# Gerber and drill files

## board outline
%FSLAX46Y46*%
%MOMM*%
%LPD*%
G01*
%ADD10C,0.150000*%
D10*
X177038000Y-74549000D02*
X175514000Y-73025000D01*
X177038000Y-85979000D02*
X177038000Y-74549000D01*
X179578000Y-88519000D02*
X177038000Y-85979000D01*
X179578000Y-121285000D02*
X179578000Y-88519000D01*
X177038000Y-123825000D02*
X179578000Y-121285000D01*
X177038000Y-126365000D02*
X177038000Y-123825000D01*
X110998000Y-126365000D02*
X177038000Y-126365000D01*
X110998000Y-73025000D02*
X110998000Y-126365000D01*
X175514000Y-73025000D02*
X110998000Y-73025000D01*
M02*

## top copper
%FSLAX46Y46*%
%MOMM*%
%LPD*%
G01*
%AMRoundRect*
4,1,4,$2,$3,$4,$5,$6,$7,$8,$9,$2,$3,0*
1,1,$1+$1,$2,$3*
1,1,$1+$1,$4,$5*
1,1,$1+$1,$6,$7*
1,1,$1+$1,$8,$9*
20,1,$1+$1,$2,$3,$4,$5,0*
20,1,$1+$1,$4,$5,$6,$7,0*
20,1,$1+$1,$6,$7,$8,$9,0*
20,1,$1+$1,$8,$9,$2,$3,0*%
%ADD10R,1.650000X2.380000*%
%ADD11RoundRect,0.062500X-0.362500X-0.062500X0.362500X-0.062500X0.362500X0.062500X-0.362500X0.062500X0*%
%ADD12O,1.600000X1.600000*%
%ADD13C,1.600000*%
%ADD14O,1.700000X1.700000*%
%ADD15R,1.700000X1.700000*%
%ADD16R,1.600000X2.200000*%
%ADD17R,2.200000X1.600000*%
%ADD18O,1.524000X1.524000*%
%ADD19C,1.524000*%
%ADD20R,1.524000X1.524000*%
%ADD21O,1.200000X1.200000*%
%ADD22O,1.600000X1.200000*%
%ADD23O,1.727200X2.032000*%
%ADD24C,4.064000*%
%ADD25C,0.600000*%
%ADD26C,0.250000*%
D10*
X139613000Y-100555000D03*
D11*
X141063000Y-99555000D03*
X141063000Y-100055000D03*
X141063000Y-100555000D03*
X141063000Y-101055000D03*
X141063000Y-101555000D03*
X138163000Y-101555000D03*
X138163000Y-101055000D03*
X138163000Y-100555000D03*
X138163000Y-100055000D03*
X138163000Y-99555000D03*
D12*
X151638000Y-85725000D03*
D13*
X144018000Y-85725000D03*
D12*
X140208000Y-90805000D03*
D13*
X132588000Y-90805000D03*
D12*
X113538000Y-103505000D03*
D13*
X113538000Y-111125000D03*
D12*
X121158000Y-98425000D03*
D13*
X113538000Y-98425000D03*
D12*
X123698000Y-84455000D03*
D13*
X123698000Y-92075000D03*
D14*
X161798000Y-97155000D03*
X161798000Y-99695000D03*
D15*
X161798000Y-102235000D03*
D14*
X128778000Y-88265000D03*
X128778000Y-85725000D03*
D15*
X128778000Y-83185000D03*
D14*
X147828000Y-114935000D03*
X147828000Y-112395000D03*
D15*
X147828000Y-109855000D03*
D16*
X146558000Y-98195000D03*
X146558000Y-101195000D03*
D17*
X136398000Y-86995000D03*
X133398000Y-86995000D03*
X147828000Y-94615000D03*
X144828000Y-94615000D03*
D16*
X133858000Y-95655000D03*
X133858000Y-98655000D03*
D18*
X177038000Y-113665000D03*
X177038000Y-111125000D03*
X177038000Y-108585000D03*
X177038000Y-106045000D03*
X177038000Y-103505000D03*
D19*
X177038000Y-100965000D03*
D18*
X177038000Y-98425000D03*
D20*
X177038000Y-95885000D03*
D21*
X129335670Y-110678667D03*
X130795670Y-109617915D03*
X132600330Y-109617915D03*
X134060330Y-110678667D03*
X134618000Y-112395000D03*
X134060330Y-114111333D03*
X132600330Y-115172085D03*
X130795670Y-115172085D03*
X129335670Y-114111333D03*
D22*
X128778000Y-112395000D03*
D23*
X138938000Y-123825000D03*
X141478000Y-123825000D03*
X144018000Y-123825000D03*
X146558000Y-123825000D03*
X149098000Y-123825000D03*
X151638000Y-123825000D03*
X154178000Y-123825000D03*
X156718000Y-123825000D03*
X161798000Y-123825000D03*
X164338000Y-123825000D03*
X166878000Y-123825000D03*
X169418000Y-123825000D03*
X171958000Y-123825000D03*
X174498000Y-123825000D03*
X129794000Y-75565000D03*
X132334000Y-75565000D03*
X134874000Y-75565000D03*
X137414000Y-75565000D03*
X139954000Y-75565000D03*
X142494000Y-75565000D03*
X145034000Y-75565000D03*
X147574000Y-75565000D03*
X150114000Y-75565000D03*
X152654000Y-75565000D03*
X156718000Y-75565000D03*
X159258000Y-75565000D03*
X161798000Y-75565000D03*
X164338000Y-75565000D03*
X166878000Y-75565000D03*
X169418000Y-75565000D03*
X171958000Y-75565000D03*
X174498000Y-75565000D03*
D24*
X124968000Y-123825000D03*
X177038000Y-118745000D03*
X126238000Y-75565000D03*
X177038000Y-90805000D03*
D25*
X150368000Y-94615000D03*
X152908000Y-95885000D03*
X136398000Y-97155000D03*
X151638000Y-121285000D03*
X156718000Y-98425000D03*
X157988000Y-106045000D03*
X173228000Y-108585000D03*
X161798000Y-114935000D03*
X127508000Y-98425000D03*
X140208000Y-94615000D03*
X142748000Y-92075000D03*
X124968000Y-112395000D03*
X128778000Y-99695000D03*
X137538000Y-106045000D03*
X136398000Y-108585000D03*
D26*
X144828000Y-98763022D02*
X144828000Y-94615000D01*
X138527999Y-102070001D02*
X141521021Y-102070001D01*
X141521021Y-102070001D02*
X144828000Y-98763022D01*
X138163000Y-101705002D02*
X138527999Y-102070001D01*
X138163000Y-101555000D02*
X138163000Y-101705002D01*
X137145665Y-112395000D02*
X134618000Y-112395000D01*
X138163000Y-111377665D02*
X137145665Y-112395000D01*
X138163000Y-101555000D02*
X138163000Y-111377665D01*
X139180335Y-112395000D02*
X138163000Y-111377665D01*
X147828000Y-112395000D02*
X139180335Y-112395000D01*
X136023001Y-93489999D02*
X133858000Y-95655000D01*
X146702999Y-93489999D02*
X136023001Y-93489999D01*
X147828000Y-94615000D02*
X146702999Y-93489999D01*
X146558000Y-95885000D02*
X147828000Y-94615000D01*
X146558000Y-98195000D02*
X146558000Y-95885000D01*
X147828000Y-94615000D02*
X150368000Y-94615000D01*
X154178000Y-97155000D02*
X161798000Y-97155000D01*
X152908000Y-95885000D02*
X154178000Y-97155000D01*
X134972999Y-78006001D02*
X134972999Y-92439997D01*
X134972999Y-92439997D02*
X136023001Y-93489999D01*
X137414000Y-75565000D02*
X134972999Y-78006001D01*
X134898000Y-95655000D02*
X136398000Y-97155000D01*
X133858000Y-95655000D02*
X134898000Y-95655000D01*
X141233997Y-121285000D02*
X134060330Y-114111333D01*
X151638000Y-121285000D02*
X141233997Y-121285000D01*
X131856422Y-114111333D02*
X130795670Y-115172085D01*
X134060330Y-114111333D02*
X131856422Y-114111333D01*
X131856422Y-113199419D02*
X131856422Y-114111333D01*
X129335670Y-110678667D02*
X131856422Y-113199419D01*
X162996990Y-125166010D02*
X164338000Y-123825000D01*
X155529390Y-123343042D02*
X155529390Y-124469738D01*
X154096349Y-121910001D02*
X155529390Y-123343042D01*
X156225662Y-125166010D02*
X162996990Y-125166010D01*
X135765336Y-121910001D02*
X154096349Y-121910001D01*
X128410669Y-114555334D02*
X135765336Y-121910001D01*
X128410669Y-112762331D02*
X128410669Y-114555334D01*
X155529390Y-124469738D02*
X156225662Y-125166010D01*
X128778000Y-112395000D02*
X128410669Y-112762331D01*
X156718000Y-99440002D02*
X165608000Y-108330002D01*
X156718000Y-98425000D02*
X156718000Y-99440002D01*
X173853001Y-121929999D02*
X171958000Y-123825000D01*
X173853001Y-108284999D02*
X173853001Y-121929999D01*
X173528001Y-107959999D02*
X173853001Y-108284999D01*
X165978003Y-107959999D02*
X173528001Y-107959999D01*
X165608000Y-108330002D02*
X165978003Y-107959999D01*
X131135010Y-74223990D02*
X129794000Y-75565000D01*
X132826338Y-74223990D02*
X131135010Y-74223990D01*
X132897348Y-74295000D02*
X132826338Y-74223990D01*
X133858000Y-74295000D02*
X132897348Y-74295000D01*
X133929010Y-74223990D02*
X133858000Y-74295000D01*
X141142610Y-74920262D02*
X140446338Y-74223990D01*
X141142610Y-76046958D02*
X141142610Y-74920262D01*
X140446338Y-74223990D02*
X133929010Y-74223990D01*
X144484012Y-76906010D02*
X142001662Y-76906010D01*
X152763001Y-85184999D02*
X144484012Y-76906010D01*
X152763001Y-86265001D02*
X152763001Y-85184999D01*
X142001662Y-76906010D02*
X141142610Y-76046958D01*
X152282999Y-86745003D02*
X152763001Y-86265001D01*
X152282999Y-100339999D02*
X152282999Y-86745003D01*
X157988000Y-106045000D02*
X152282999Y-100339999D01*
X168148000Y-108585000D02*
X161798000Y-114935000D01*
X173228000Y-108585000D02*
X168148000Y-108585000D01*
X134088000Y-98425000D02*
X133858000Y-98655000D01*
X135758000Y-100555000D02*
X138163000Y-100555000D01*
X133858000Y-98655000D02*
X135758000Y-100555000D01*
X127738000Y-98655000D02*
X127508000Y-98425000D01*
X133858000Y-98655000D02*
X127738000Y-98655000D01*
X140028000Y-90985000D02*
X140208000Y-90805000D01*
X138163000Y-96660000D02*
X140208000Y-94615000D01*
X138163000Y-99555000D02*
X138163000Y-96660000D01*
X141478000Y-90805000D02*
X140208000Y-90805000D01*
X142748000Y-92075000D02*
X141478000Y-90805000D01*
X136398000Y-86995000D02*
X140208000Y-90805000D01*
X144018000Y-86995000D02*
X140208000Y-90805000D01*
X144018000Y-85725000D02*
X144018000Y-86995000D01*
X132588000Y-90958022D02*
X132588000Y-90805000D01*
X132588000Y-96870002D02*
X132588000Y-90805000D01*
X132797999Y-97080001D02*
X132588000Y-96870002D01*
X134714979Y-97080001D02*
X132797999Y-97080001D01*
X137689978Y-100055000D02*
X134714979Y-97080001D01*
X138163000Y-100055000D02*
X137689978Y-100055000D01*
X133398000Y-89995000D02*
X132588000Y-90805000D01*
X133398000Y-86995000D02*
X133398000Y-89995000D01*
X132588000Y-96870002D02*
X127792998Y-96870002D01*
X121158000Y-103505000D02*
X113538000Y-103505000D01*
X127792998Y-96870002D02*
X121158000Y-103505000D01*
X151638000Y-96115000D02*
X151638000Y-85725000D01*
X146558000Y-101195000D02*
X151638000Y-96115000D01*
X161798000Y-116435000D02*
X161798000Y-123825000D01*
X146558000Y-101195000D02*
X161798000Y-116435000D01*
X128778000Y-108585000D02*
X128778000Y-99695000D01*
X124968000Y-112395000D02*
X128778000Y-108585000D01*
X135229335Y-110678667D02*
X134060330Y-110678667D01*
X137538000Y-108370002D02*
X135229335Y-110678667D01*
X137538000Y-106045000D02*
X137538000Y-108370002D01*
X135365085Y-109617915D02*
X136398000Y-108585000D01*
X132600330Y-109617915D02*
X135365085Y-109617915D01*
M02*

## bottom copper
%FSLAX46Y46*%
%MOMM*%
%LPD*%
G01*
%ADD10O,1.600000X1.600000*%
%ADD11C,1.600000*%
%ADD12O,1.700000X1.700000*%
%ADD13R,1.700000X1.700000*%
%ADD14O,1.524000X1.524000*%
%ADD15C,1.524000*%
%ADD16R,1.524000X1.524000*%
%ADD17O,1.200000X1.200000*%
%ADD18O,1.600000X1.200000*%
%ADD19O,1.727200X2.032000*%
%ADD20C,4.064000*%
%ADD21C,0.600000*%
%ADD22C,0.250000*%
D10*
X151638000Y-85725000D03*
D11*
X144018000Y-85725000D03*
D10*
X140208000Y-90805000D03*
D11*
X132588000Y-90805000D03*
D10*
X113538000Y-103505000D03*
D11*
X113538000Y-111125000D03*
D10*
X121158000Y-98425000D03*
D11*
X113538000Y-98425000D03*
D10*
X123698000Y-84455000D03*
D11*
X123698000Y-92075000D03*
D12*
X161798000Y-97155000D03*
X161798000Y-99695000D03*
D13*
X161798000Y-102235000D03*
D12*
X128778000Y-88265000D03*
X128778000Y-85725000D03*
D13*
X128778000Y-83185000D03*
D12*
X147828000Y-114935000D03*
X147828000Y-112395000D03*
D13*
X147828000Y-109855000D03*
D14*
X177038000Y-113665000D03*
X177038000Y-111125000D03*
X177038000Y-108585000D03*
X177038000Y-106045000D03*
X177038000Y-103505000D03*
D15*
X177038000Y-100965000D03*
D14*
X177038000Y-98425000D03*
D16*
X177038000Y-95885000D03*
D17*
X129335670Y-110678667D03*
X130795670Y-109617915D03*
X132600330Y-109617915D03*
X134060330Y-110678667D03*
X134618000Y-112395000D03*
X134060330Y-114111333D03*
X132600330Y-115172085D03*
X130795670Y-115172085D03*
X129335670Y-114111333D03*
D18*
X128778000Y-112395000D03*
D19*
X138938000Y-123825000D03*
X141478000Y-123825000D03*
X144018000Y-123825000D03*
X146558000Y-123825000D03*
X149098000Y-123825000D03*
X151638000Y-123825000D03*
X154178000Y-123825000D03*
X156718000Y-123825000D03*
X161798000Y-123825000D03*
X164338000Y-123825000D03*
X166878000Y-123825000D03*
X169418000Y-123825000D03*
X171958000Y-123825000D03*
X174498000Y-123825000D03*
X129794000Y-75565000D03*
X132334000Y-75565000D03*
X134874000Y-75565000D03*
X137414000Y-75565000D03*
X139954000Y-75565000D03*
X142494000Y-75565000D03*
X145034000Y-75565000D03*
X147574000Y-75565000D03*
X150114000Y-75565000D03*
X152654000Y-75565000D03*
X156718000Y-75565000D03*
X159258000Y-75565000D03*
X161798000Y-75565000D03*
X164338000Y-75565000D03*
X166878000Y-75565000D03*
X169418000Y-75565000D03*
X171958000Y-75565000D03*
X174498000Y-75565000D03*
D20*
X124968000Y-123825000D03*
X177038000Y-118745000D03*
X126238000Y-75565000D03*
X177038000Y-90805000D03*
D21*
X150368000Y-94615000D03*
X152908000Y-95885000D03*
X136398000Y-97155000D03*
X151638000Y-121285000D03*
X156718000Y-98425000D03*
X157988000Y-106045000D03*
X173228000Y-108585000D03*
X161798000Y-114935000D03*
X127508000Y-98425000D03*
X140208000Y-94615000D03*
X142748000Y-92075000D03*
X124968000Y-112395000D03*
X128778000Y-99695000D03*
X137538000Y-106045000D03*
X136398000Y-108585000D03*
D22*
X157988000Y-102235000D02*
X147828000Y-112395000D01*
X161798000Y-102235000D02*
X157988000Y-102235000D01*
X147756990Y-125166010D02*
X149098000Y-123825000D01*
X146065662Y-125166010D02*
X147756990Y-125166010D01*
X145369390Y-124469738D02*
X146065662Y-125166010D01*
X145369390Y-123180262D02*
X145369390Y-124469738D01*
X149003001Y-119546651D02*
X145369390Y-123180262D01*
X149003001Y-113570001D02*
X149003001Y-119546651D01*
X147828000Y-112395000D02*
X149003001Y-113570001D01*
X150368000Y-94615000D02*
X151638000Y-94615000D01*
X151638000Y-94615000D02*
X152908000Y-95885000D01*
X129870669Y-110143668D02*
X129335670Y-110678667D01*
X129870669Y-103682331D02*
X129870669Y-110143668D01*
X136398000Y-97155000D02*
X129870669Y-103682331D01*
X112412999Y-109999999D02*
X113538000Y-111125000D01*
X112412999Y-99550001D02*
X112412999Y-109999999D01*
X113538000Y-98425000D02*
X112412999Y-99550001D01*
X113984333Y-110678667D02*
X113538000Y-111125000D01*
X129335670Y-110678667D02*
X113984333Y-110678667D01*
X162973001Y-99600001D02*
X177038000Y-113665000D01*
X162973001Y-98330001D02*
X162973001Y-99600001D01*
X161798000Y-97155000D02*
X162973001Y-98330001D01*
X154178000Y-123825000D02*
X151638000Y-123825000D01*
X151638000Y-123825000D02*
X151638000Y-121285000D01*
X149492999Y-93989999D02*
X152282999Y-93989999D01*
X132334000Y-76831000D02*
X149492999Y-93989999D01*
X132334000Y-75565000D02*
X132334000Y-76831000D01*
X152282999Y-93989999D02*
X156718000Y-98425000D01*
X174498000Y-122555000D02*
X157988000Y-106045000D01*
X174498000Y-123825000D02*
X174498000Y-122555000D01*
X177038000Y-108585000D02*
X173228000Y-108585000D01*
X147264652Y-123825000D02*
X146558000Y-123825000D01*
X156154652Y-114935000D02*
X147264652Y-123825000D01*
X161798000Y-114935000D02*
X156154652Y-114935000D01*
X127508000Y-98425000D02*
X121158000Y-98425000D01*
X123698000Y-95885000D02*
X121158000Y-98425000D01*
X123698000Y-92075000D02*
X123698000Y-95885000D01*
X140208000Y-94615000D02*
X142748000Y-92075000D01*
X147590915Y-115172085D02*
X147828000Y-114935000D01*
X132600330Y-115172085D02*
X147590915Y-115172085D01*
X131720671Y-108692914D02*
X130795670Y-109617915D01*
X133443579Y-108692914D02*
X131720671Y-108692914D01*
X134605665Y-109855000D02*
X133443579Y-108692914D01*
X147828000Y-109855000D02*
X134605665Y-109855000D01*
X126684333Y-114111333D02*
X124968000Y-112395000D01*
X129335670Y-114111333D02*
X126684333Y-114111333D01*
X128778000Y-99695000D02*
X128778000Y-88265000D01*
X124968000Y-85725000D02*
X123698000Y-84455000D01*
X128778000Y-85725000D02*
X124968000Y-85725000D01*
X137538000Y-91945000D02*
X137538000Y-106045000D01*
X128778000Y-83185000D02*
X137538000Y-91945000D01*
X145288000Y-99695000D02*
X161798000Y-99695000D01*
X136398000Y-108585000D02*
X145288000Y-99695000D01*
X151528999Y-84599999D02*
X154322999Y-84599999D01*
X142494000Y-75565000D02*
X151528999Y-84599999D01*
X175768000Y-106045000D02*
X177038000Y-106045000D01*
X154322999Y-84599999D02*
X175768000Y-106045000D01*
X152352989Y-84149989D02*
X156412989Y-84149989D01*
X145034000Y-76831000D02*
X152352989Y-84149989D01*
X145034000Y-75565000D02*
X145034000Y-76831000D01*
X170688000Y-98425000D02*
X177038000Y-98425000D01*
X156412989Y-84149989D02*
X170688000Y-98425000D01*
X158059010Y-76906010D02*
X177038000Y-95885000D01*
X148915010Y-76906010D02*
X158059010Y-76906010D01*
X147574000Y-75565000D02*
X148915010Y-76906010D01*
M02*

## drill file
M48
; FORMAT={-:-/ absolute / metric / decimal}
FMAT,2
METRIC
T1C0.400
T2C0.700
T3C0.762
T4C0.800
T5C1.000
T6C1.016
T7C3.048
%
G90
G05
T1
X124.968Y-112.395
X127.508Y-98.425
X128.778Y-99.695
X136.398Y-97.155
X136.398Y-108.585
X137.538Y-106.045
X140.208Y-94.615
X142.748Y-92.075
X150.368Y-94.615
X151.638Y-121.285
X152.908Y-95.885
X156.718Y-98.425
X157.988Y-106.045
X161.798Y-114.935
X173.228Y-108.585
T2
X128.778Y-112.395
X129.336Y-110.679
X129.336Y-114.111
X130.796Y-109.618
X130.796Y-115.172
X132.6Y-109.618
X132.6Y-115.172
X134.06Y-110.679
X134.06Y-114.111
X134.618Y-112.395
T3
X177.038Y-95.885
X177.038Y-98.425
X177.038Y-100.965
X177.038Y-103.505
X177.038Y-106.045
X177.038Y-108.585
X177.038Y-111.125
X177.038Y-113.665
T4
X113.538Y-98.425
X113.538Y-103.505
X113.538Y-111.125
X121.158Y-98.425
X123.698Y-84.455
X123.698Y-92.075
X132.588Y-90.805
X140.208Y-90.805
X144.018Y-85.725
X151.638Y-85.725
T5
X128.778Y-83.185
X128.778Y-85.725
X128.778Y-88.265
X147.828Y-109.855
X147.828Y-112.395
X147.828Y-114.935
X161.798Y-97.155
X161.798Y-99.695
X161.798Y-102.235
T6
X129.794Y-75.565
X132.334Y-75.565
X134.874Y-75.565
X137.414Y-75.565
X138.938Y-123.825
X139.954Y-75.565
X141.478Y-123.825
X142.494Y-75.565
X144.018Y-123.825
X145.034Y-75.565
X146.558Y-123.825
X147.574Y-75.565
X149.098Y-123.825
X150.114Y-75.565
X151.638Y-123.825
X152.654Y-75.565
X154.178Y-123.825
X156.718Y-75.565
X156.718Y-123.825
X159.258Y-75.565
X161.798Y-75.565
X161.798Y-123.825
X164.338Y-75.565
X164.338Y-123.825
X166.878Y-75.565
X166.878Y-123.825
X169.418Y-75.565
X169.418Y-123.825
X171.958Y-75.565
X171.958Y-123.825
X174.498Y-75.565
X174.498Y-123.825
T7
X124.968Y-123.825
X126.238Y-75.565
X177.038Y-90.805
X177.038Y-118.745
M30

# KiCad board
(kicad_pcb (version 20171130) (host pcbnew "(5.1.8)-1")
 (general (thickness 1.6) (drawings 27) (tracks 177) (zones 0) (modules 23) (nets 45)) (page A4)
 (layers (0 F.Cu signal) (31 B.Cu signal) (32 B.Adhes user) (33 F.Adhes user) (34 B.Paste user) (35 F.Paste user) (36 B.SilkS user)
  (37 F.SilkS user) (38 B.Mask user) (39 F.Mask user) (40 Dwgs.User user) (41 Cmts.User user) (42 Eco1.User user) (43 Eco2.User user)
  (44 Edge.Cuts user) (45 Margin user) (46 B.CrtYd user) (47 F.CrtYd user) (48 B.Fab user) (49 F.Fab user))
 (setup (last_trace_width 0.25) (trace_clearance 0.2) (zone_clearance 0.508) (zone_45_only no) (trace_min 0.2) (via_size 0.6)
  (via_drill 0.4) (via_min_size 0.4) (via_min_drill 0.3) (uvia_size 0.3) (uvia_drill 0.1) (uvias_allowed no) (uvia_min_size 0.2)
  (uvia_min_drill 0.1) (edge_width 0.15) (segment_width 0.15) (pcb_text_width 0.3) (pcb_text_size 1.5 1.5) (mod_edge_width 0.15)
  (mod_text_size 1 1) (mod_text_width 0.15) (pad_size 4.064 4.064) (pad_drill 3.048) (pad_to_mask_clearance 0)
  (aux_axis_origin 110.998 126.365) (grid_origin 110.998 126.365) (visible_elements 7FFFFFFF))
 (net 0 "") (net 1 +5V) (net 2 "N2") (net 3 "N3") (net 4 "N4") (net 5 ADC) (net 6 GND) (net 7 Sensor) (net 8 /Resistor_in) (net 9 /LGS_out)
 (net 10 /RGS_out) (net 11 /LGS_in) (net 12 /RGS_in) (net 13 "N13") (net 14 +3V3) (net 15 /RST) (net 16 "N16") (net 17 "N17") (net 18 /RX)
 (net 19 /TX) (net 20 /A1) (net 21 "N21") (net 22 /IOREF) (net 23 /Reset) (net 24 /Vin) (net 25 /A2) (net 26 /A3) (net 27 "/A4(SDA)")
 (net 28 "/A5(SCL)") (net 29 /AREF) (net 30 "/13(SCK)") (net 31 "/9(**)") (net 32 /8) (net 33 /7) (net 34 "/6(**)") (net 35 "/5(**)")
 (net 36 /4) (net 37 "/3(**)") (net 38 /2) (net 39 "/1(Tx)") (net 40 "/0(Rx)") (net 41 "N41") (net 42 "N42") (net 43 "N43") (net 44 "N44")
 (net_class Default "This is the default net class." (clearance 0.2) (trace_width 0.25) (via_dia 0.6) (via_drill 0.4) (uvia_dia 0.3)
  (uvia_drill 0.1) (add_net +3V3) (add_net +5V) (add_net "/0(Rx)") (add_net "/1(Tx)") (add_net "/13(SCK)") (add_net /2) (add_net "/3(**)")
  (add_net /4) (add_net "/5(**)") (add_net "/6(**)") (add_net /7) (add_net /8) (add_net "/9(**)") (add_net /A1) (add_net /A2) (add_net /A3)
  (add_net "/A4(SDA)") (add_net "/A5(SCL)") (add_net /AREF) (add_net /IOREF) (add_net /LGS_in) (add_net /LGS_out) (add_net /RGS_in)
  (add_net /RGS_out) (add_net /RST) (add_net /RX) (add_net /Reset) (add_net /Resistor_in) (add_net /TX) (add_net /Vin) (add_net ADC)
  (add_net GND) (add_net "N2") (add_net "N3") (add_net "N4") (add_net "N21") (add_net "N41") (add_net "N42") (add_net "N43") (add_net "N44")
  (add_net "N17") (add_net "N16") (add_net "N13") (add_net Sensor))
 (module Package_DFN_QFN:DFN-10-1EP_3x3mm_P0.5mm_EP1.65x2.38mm (layer F.Cu) (at 139.613 100.555)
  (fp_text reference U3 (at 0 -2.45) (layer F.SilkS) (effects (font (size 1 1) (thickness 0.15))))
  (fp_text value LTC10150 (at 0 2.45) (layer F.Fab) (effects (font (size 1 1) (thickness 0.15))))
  (pad "" smd roundrect (at 0.41 0.595) (size 0.67 0.96) (layers F.Paste) (roundrect_rratio 0.25))
  (pad "" smd roundrect (at 0.41 -0.595) (size 0.67 0.96) (layers F.Paste) (roundrect_rratio 0.25))
  (pad "" smd roundrect (at -0.41 0.595) (size 0.67 0.96) (layers F.Paste) (roundrect_rratio 0.25))
  (pad "" smd roundrect (at -0.41 -0.595) (size 0.67 0.96) (layers F.Paste) (roundrect_rratio 0.25))
  (pad 11 smd rect (at 0 0) (size 1.65 2.38) (layers F.Cu F.Mask))
  (pad 10 smd roundrect (at 1.45 -1) (size 0.85 0.25) (layers F.Cu F.Paste F.Mask) (roundrect_rratio 0.25))
  (pad 9 smd roundrect (at 1.45 -0.5) (size 0.85 0.25) (layers F.Cu F.Paste F.Mask) (roundrect_rratio 0.25))
  (pad 8 smd roundrect (at 1.45 0) (size 0.85 0.25) (layers F.Cu F.Paste F.Mask) (roundrect_rratio 0.25))
  (pad 7 smd roundrect (at 1.45 0.5) (size 0.85 0.25) (layers F.Cu F.Paste F.Mask) (roundrect_rratio 0.25))
  (pad 6 smd roundrect (at 1.45 1) (size 0.85 0.25) (layers F.Cu F.Paste F.Mask) (roundrect_rratio 0.25))
  (pad 5 smd roundrect (at -1.45 1) (size 0.85 0.25) (layers F.Cu F.Paste F.Mask) (roundrect_rratio 0.25) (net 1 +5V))
  (pad 4 smd roundrect (at -1.45 0.5) (size 0.85 0.25) (layers F.Cu F.Paste F.Mask) (roundrect_rratio 0.25))
  (pad 3 smd roundrect (at -1.45 0) (size 0.85 0.25) (layers F.Cu F.Paste F.Mask) (roundrect_rratio 0.25) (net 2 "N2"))
  (pad 2 smd roundrect (at -1.45 -0.5) (size 0.85 0.25) (layers F.Cu F.Paste F.Mask) (roundrect_rratio 0.25) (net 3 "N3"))
  (pad 1 smd roundrect (at -1.45 -1) (size 0.85 0.25) (layers F.Cu F.Paste F.Mask) (roundrect_rratio 0.25) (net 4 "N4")))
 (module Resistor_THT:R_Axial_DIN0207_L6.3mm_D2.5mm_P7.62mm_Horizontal (layer F.Cu) (at 144.018 85.725)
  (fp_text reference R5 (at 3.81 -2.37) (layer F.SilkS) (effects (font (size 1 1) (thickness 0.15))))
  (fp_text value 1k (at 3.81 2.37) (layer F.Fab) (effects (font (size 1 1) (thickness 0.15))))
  (pad 2 thru_hole oval (at 7.62 0) (size 1.6 1.6) (drill 0.8) (layers *.Cu *.Mask) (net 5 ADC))
  (pad 1 thru_hole circle (at 0 0) (size 1.6 1.6) (drill 0.8) (layers *.Cu *.Mask) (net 4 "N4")))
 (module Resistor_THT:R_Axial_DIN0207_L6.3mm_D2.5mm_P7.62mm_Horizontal (layer F.Cu) (at 132.588 90.805)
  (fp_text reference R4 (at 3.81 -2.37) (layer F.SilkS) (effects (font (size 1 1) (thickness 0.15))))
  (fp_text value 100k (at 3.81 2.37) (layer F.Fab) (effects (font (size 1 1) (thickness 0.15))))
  (pad 2 thru_hole oval (at 7.62 0) (size 1.6 1.6) (drill 0.8) (layers *.Cu *.Mask) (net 4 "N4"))
  (pad 1 thru_hole circle (at 0 0) (size 1.6 1.6) (drill 0.8) (layers *.Cu *.Mask) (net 3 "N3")))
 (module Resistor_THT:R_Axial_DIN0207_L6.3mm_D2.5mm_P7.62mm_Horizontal (layer F.Cu) (at 113.538 111.125 90)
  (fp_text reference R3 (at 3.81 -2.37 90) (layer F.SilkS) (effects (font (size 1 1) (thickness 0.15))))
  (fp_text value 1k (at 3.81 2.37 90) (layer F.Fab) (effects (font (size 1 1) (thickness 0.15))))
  (pad 2 thru_hole oval (at 7.62 0 90) (size 1.6 1.6) (drill 0.8) (layers *.Cu *.Mask) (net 3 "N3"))
  (pad 1 thru_hole circle (at 0 0 90) (size 1.6 1.6) (drill 0.8) (layers *.Cu *.Mask) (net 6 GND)))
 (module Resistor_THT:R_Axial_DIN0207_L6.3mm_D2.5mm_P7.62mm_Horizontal (layer F.Cu) (at 113.538 98.425)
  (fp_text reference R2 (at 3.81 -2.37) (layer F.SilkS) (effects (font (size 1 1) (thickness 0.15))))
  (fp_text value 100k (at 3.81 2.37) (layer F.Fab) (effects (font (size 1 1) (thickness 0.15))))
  (pad 2 thru_hole oval (at 7.62 0) (size 1.6 1.6) (drill 0.8) (layers *.Cu *.Mask) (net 2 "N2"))
  (pad 1 thru_hole circle (at 0 0) (size 1.6 1.6) (drill 0.8) (layers *.Cu *.Mask) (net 6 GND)))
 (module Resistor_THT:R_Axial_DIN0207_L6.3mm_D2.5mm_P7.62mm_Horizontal (layer F.Cu) (at 123.698 92.075 90)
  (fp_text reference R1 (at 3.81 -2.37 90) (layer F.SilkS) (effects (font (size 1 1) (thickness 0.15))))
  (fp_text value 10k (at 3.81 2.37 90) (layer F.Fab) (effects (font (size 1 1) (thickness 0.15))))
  (pad 2 thru_hole oval (at 7.62 0 90) (size 1.6 1.6) (drill 0.8) (layers *.Cu *.Mask) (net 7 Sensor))
  (pad 1 thru_hole circle (at 0 0 90) (size 1.6 1.6) (drill 0.8) (layers *.Cu *.Mask) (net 2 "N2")))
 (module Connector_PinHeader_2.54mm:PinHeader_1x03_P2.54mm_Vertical (layer F.Cu) (at 161.798 102.235 180)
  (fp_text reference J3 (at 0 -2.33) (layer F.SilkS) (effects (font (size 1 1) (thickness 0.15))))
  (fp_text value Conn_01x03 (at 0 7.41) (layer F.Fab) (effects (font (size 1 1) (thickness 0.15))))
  (pad 3 thru_hole oval (at 0 5.08 180) (size 1.7 1.7) (drill 1) (layers *.Cu *.Mask) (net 6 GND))
  (pad 2 thru_hole oval (at 0 2.54 180) (size 1.7 1.7) (drill 1) (layers *.Cu *.Mask) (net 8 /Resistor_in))
  (pad 1 thru_hole rect (at 0 0 180) (size 1.7 1.7) (drill 1) (layers *.Cu *.Mask) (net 1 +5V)))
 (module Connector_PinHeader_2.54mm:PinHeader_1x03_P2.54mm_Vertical (layer F.Cu) (at 128.778 83.185)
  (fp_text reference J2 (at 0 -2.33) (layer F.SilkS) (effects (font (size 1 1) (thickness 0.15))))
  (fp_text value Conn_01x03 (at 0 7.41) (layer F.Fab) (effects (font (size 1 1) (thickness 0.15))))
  (pad 3 thru_hole oval (at 0 5.08) (size 1.7 1.7) (drill 1) (layers *.Cu *.Mask) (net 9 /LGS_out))
  (pad 2 thru_hole oval (at 0 2.54) (size 1.7 1.7) (drill 1) (layers *.Cu *.Mask) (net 7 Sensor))
  (pad 1 thru_hole rect (at 0 0) (size 1.7 1.7) (drill 1) (layers *.Cu *.Mask) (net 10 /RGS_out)))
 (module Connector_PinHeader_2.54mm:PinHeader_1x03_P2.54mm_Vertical (layer F.Cu) (at 147.828 109.855)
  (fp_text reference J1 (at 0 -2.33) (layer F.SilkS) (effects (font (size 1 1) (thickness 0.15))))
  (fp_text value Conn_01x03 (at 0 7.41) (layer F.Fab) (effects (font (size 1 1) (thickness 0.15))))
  (pad 3 thru_hole oval (at 0 5.08) (size 1.7 1.7) (drill 1) (layers *.Cu *.Mask) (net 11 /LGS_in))
  (pad 2 thru_hole oval (at 0 2.54) (size 1.7 1.7) (drill 1) (layers *.Cu *.Mask) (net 1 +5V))
  (pad 1 thru_hole rect (at 0 0) (size 1.7 1.7) (drill 1) (layers *.Cu *.Mask) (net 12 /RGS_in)))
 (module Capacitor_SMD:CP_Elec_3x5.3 (layer F.Cu) (at 146.558 99.695 90)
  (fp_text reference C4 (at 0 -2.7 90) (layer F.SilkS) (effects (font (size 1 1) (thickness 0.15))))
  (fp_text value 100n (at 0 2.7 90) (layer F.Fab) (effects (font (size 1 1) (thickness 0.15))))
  (pad 2 smd rect (at 1.5 0 90) (size 2.2 1.6) (layers F.Cu F.Paste F.Mask) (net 6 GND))
  (pad 1 smd rect (at -1.5 0 90) (size 2.2 1.6) (layers F.Cu F.Paste F.Mask) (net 5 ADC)))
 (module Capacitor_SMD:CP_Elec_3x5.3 (layer F.Cu) (at 134.898 86.995)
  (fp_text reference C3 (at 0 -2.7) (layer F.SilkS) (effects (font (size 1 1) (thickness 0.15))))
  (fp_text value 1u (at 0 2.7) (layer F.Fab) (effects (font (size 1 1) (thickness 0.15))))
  (pad 2 smd rect (at 1.5 0) (size 2.2 1.6) (layers F.Cu F.Paste F.Mask) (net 4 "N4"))
  (pad 1 smd rect (at -1.5 0) (size 2.2 1.6) (layers F.Cu F.Paste F.Mask) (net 3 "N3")))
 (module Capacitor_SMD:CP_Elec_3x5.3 (layer F.Cu) (at 146.328 94.615)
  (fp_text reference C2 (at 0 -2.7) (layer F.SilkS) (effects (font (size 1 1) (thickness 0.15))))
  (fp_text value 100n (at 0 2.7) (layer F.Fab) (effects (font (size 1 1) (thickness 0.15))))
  (pad 2 smd rect (at 1.5 0) (size 2.2 1.6) (layers F.Cu F.Paste F.Mask) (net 6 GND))
  (pad 1 smd rect (at -1.5 0) (size 2.2 1.6) (layers F.Cu F.Paste F.Mask) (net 1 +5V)))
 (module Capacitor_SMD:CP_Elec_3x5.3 (layer F.Cu) (at 133.858 97.155 90)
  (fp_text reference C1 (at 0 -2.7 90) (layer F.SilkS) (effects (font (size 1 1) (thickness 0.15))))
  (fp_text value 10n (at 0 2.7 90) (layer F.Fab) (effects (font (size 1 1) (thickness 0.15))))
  (pad 2 smd rect (at 1.5 0 90) (size 2.2 1.6) (layers F.Cu F.Paste F.Mask) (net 6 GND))
  (pad 1 smd rect (at -1.5 0 90) (size 2.2 1.6) (layers F.Cu F.Paste F.Mask) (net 2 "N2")))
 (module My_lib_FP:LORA (layer F.Cu) (at 197.358 106.045 270)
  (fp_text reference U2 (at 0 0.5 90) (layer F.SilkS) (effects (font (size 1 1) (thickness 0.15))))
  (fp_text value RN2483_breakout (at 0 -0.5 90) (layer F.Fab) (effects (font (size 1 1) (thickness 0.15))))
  (pad 8 thru_hole oval (at 7.62 20.32 270) (size 1.524 1.524) (drill 0.762) (layers *.Cu *.Mask) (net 6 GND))
  (pad 7 thru_hole oval (at 5.08 20.32 270) (size 1.524 1.524) (drill 0.762) (layers *.Cu *.Mask) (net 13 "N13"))
  (pad 6 thru_hole oval (at 2.54 20.32 270) (size 1.524 1.524) (drill 0.762) (layers *.Cu *.Mask) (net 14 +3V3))
  (pad 5 thru_hole oval (at 0 20.32 270) (size 1.524 1.524) (drill 0.762) (layers *.Cu *.Mask) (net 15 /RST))
  (pad 4 thru_hole oval (at -2.54 20.32 270) (size 1.524 1.524) (drill 0.762) (layers *.Cu *.Mask) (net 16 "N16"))
  (pad 3 thru_hole circle (at -5.08 20.32 270) (size 1.524 1.524) (drill 0.762) (layers *.Cu *.Mask) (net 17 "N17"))
  (pad 2 thru_hole oval (at -7.62 20.32 270) (size 1.524 1.524) (drill 0.762) (layers *.Cu *.Mask B.Adhes) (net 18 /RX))
  (pad 1 thru_hole rect (at -10.16 20.32 270) (size 1.524 1.524) (drill 0.762) (layers *.Cu *.Mask) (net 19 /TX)))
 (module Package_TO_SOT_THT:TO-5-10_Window (layer F.Cu) (at 128.778 112.395)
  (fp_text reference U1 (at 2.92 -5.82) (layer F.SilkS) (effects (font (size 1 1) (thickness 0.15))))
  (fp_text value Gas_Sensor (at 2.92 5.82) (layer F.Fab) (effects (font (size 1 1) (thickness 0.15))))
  (pad 10 thru_hole oval (at 0.55767 -1.716333) (size 1.2 1.2) (drill 0.7) (layers *.Cu *.Mask) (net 6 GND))
  (pad 9 thru_hole oval (at 2.01767 -2.777085) (size 1.2 1.2) (drill 0.7) (layers *.Cu *.Mask) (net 12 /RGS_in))
  (pad 8 thru_hole oval (at 3.82233 -2.777085) (size 1.2 1.2) (drill 0.7) (layers *.Cu *.Mask) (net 8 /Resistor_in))
  (pad 7 thru_hole oval (at 5.28233 -1.716333) (size 1.2 1.2) (drill 0.7) (layers *.Cu *.Mask) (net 10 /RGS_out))
  (pad 6 thru_hole oval (at 5.84 0) (size 1.2 1.2) (drill 0.7) (layers *.Cu *.Mask) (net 1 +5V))
  (pad 5 thru_hole oval (at 5.28233 1.716333) (size 1.2 1.2) (drill 0.7) (layers *.Cu *.Mask) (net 6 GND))
  (pad 4 thru_hole oval (at 3.82233 2.777085) (size 1.2 1.2) (drill 0.7) (layers *.Cu *.Mask) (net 11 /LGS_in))
  (pad 3 thru_hole oval (at 2.01767 2.777085) (size 1.2 1.2) (drill 0.7) (layers *.Cu *.Mask) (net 6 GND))
  (pad 2 thru_hole oval (at 0.55767 1.716333) (size 1.2 1.2) (drill 0.7) (layers *.Cu *.Mask) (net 9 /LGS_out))
  (pad 1 thru_hole oval (at 0 0) (size 1.6 1.2) (drill 0.7) (layers *.Cu *.Mask) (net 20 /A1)))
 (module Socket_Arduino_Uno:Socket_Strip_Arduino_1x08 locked (layer F.Cu) (at 138.938 123.825)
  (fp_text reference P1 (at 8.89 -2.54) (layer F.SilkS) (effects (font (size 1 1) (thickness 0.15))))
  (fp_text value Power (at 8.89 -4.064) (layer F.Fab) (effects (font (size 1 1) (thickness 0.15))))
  (pad 1 thru_hole oval (at 0 0) (size 1.7272 2.032) (drill 1.016) (layers *.Cu *.Mask F.SilkS) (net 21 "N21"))
  (pad 2 thru_hole oval (at 2.54 0) (size 1.7272 2.032) (drill 1.016) (layers *.Cu *.Mask F.SilkS) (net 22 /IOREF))
  (pad 3 thru_hole oval (at 5.08 0) (size 1.7272 2.032) (drill 1.016) (layers *.Cu *.Mask F.SilkS) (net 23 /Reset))
  (pad 4 thru_hole oval (at 7.62 0) (size 1.7272 2.032) (drill 1.016) (layers *.Cu *.Mask F.SilkS) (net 14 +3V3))
  (pad 5 thru_hole oval (at 10.16 0) (size 1.7272 2.032) (drill 1.016) (layers *.Cu *.Mask F.SilkS) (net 1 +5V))
  (pad 6 thru_hole oval (at 12.7 0) (size 1.7272 2.032) (drill 1.016) (layers *.Cu *.Mask F.SilkS) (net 6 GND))
  (pad 7 thru_hole oval (at 15.24 0) (size 1.7272 2.032) (drill 1.016) (layers *.Cu *.Mask F.SilkS) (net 6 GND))
  (pad 8 thru_hole oval (at 17.78 0) (size 1.7272 2.032) (drill 1.016) (layers *.Cu *.Mask F.SilkS) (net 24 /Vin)))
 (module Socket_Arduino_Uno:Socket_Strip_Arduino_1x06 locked (layer F.Cu) (at 161.798 123.825)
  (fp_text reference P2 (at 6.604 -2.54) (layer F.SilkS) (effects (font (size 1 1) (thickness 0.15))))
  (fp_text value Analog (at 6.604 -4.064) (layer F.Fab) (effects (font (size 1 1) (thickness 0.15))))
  (pad 1 thru_hole oval (at 0 0) (size 1.7272 2.032) (drill 1.016) (layers *.Cu *.Mask F.SilkS) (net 5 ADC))
  (pad 2 thru_hole oval (at 2.54 0) (size 1.7272 2.032) (drill 1.016) (layers *.Cu *.Mask F.SilkS) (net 20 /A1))
  (pad 3 thru_hole oval (at 5.08 0) (size 1.7272 2.032) (drill 1.016) (layers *.Cu *.Mask F.SilkS) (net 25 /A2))
  (pad 4 thru_hole oval (at 7.62 0) (size 1.7272 2.032) (drill 1.016) (layers *.Cu *.Mask F.SilkS) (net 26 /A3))
  (pad 5 thru_hole oval (at 10.16 0) (size 1.7272 2.032) (drill 1.016) (layers *.Cu *.Mask F.SilkS) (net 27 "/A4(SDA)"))
  (pad 6 thru_hole oval (at 12.7 0) (size 1.7272 2.032) (drill 1.016) (layers *.Cu *.Mask F.SilkS) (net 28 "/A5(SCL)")))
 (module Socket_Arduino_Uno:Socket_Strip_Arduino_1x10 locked (layer F.Cu) (at 129.794 75.565)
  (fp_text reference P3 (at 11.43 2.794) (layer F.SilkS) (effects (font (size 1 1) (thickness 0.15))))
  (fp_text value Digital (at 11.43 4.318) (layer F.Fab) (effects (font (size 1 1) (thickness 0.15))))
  (pad 1 thru_hole oval (at 0 0) (size 1.7272 2.032) (drill 1.016) (layers *.Cu *.Mask F.SilkS) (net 28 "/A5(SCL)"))
  (pad 2 thru_hole oval (at 2.54 0) (size 1.7272 2.032) (drill 1.016) (layers *.Cu *.Mask F.SilkS) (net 27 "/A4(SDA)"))
  (pad 3 thru_hole oval (at 5.08 0) (size 1.7272 2.032) (drill 1.016) (layers *.Cu *.Mask F.SilkS) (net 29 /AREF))
  (pad 4 thru_hole oval (at 7.62 0) (size 1.7272 2.032) (drill 1.016) (layers *.Cu *.Mask F.SilkS) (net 6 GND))
  (pad 5 thru_hole oval (at 10.16 0) (size 1.7272 2.032) (drill 1.016) (layers *.Cu *.Mask F.SilkS) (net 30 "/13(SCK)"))
  (pad 6 thru_hole oval (at 12.7 0) (size 1.7272 2.032) (drill 1.016) (layers *.Cu *.Mask F.SilkS) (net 15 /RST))
  (pad 7 thru_hole oval (at 15.24 0) (size 1.7272 2.032) (drill 1.016) (layers *.Cu *.Mask F.SilkS) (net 18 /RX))
  (pad 8 thru_hole oval (at 17.78 0) (size 1.7272 2.032) (drill 1.016) (layers *.Cu *.Mask F.SilkS) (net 19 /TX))
  (pad 9 thru_hole oval (at 20.32 0) (size 1.7272 2.032) (drill 1.016) (layers *.Cu *.Mask F.SilkS) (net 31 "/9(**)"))
  (pad 10 thru_hole oval (at 22.86 0) (size 1.7272 2.032) (drill 1.016) (layers *.Cu *.Mask F.SilkS) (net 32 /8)))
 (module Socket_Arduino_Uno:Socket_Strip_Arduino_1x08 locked (layer F.Cu) (at 156.718 75.565)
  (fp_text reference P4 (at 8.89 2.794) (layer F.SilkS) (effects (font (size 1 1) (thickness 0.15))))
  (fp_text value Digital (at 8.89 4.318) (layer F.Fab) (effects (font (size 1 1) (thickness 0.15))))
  (pad 1 thru_hole oval (at 0 0) (size 1.7272 2.032) (drill 1.016) (layers *.Cu *.Mask F.SilkS) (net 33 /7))
  (pad 2 thru_hole oval (at 2.54 0) (size 1.7272 2.032) (drill 1.016) (layers *.Cu *.Mask F.SilkS) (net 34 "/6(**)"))
  (pad 3 thru_hole oval (at 5.08 0) (size 1.7272 2.032) (drill 1.016) (layers *.Cu *.Mask F.SilkS) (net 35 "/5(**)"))
  (pad 4 thru_hole oval (at 7.62 0) (size 1.7272 2.032) (drill 1.016) (layers *.Cu *.Mask F.SilkS) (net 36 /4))
  (pad 5 thru_hole oval (at 10.16 0) (size 1.7272 2.032) (drill 1.016) (layers *.Cu *.Mask F.SilkS) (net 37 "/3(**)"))
  (pad 6 thru_hole oval (at 12.7 0) (size 1.7272 2.032) (drill 1.016) (layers *.Cu *.Mask F.SilkS) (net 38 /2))
  (pad 7 thru_hole oval (at 15.24 0) (size 1.7272 2.032) (drill 1.016) (layers *.Cu *.Mask F.SilkS) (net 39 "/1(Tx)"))
  (pad 8 thru_hole oval (at 17.78 0) (size 1.7272 2.032) (drill 1.016) (layers *.Cu *.Mask F.SilkS) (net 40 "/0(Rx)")))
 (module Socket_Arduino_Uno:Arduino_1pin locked (layer F.Cu) (at 124.968 123.825)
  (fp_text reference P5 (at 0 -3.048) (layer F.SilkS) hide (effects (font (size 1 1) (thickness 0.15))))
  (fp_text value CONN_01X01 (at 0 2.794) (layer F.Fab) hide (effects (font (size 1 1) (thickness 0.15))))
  (pad 1 thru_hole circle (at 0 0) (size 4.064 4.064) (drill 3.048) (layers *.Cu *.Mask F.SilkS) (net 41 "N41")))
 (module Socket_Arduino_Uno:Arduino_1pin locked (layer F.Cu) (at 177.038 118.745)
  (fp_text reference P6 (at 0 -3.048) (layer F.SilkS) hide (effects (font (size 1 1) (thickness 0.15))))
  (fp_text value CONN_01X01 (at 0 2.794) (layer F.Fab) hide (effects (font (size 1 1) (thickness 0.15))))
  (pad 1 thru_hole circle (at 0 0) (size 4.064 4.064) (drill 3.048) (layers *.Cu *.Mask F.SilkS) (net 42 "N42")))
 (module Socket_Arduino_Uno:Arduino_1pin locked (layer F.Cu) (at 126.238 75.565)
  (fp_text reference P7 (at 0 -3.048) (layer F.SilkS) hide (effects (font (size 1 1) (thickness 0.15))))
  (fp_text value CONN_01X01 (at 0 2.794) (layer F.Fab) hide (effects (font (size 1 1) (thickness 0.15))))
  (pad 1 thru_hole circle (at 0 0) (size 4.064 4.064) (drill 3.048) (layers *.Cu *.Mask F.SilkS) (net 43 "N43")))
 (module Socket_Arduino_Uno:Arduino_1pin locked (layer F.Cu) (at 177.038 90.805)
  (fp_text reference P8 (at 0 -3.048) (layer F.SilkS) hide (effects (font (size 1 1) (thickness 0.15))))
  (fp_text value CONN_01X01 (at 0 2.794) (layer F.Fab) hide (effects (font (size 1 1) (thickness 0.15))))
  (pad 1 thru_hole circle (at 0 0) (size 4.064 4.064) (drill 3.048) (layers *.Cu *.Mask F.SilkS) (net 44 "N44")))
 (gr_line (start 177.038 74.549) (end 175.514 73.025) (angle 90) (layer Edge.Cuts) (width 0.15))
 (gr_line (start 177.038 85.979) (end 177.038 74.549) (angle 90) (layer Edge.Cuts) (width 0.15))
 (gr_line (start 179.578 88.519) (end 177.038 85.979) (angle 90) (layer Edge.Cuts) (width 0.15))
 (gr_line (start 179.578 121.285) (end 179.578 88.519) (angle 90) (layer Edge.Cuts) (width 0.15))
 (gr_line (start 177.038 123.825) (end 179.578 121.285) (angle 90) (layer Edge.Cuts) (width 0.15))
 (gr_line (start 177.038 126.365) (end 177.038 123.825) (angle 90) (layer Edge.Cuts) (width 0.15))
 (gr_line (start 110.998 126.365) (end 177.038 126.365) (angle 90) (layer Edge.Cuts) (width 0.15))
 (gr_line (start 110.998 73.025) (end 110.998 126.365) (angle 90) (layer Edge.Cuts) (width 0.15))
 (gr_line (start 175.514 73.025) (end 110.998 73.025) (angle 90) (layer Edge.Cuts) (width 0.15))
 (segment (start 144.828 98.763022) (end 144.828 94.615) (width 0.25) (layer F.Cu) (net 1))
 (segment (start 138.527999 102.070001) (end 141.521021 102.070001) (width 0.25) (layer F.Cu) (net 1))
 (segment (start 141.521021 102.070001) (end 144.828 98.763022) (width 0.25) (layer F.Cu) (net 1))
 (segment (start 138.163 101.705002) (end 138.527999 102.070001) (width 0.25) (layer F.Cu) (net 1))
 (segment (start 138.163 101.555) (end 138.163 101.705002) (width 0.25) (layer F.Cu) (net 1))
 (segment (start 137.145665 112.395) (end 134.618 112.395) (width 0.25) (layer F.Cu) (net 1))
 (segment (start 138.163 111.377665) (end 137.145665 112.395) (width 0.25) (layer F.Cu) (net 1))
 (segment (start 138.163 101.555) (end 138.163 111.377665) (width 0.25) (layer F.Cu) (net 1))
 (segment (start 157.988 102.235) (end 147.828 112.395) (width 0.25) (layer B.Cu) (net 1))
 (segment (start 161.798 102.235) (end 157.988 102.235) (width 0.25) (layer B.Cu) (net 1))
 (segment (start 139.180335 112.395) (end 138.163 111.377665) (width 0.25) (layer F.Cu) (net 1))
 (segment (start 147.828 112.395) (end 139.180335 112.395) (width 0.25) (layer F.Cu) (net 1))
 (segment (start 147.75699 125.16601) (end 149.098 123.825) (width 0.25) (layer B.Cu) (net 1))
 (segment (start 146.065662 125.16601) (end 147.75699 125.16601) (width 0.25) (layer B.Cu) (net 1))
 (segment (start 145.36939 124.469738) (end 146.065662 125.16601) (width 0.25) (layer B.Cu) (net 1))
 (segment (start 145.36939 123.180262) (end 145.36939 124.469738) (width 0.25) (layer B.Cu) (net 1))
 (segment (start 149.003001 119.546651) (end 145.36939 123.180262) (width 0.25) (layer B.Cu) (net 1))
 (segment (start 149.003001 113.570001) (end 149.003001 119.546651) (width 0.25) (layer B.Cu) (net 1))
 (segment (start 147.828 112.395) (end 149.003001 113.570001) (width 0.25) (layer B.Cu) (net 1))
 (segment (start 136.023001 93.489999) (end 133.858 95.655) (width 0.25) (layer F.Cu) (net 6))
 (segment (start 146.702999 93.489999) (end 136.023001 93.489999) (width 0.25) (layer F.Cu) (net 6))
 (segment (start 147.828 94.615) (end 146.702999 93.489999) (width 0.25) (layer F.Cu) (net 6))
 (segment (start 146.558 95.885) (end 147.828 94.615) (width 0.25) (layer F.Cu) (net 6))
 (segment (start 146.558 98.195) (end 146.558 95.885) (width 0.25) (layer F.Cu) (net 6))
 (via (at 150.368 94.615) (size 0.6) (drill 0.4) (layers F.Cu B.Cu) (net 6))
 (segment (start 147.828 94.615) (end 150.368 94.615) (width 0.25) (layer F.Cu) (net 6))
 (segment (start 150.368 94.615) (end 151.638 94.615) (width 0.25) (layer B.Cu) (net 6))
 (via (at 152.908 95.885) (size 0.6) (drill 0.4) (layers F.Cu B.Cu) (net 6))
 (segment (start 151.638 94.615) (end 152.908 95.885) (width 0.25) (layer B.Cu) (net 6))
 (segment (start 154.178 97.155) (end 161.798 97.155) (width 0.25) (layer F.Cu) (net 6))
 (segment (start 152.908 95.885) (end 154.178 97.155) (width 0.25) (layer F.Cu) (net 6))
 (segment (start 134.972999 78.006001) (end 134.972999 92.439997) (width 0.25) (layer F.Cu) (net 6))
 (segment (start 134.972999 92.439997) (end 136.023001 93.489999) (width 0.25) (layer F.Cu) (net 6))
 (segment (start 137.414 75.565) (end 134.972999 78.006001) (width 0.25) (layer F.Cu) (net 6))
 (via (at 136.398 97.155) (size 0.6) (drill 0.4) (layers F.Cu B.Cu) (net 6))
 (segment (start 134.898 95.655) (end 136.398 97.155) (width 0.25) (layer F.Cu) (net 6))
 (segment (start 133.858 95.655) (end 134.898 95.655) (width 0.25) (layer F.Cu) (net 6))
 (segment (start 129.870669 110.143668) (end 129.33567 110.678667) (width 0.25) (layer B.Cu) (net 6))
 (segment (start 129.870669 103.682331) (end 129.870669 110.143668) (width 0.25) (layer B.Cu) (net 6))
 (segment (start 136.398 97.155) (end 129.870669 103.682331) (width 0.25) (layer B.Cu) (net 6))
 (segment (start 112.412999 109.999999) (end 113.538 111.125) (width 0.25) (layer B.Cu) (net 6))
 (segment (start 112.412999 99.550001) (end 112.412999 109.999999) (width 0.25) (layer B.Cu) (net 6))
 (segment (start 113.538 98.425) (end 112.412999 99.550001) (width 0.25) (layer B.Cu) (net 6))
 (segment (start 113.984333 110.678667) (end 113.538 111.125) (width 0.25) (layer B.Cu) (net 6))
 (segment (start 129.33567 110.678667) (end 113.984333 110.678667) (width 0.25) (layer B.Cu) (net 6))
 (segment (start 162.973001 99.600001) (end 177.038 113.665) (width 0.25) (layer B.Cu) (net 6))
 (segment (start 162.973001 98.330001) (end 162.973001 99.600001) (width 0.25) (layer B.Cu) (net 6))
 (segment (start 161.798 97.155) (end 162.973001 98.330001) (width 0.25) (layer B.Cu) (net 6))
 (segment (start 154.178 123.825) (end 151.638 123.825) (width 0.25) (layer B.Cu) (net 6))
 (via (at 151.638 121.285) (size 0.6) (drill 0.4) (layers F.Cu B.Cu) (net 6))
 (segment (start 151.638 123.825) (end 151.638 121.285) (width 0.25) (layer B.Cu) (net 6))
 (segment (start 141.233997 121.285) (end 134.06033 114.111333) (width 0.25) (layer F.Cu) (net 6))
 (segment (start 151.638 121.285) (end 141.233997 121.285) (width 0.25) (layer F.Cu) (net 6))
 (segment (start 131.856422 114.111333) (end 130.79567 115.172085) (width 0.25) (layer F.Cu) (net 6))
 (segment (start 134.06033 114.111333) (end 131.856422 114.111333) (width 0.25) (layer F.Cu) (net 6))
 (segment (start 131.856422 113.199419) (end 131.856422 114.111333) (width 0.25) (layer F.Cu) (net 6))
 (segment (start 129.33567 110.678667) (end 131.856422 113.199419) (width 0.25) (layer F.Cu) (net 6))
 (segment (start 162.99699 125.16601) (end 164.338 123.825) (width 0.25) (layer F.Cu) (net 20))
 (segment (start 155.52939 123.343042) (end 155.52939 124.469738) (width 0.25) (layer F.Cu) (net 20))
 (segment (start 154.096349 121.910001) (end 155.52939 123.343042) (width 0.25) (layer F.Cu) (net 20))
 (segment (start 156.225662 125.16601) (end 162.99699 125.16601) (width 0.25) (layer F.Cu) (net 20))
 (segment (start 135.765336 121.910001) (end 154.096349 121.910001) (width 0.25) (layer F.Cu) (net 20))
 (segment (start 128.410669 114.555334) (end 135.765336 121.910001) (width 0.25) (layer F.Cu) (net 20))
 (segment (start 128.410669 112.762331) (end 128.410669 114.555334) (width 0.25) (layer F.Cu) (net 20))
 (segment (start 155.52939 124.469738) (end 156.225662 125.16601) (width 0.25) (layer F.Cu) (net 20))
 (segment (start 128.778 112.395) (end 128.410669 112.762331) (width 0.25) (layer F.Cu) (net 20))
 (segment (start 149.492999 93.989999) (end 152.282999 93.989999) (width 0.25) (layer B.Cu) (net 27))
 (segment (start 132.334 76.831) (end 149.492999 93.989999) (width 0.25) (layer B.Cu) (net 27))
 (segment (start 132.334 75.565) (end 132.334 76.831) (width 0.25) (layer B.Cu) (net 27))
 (via (at 156.718 98.425) (size 0.6) (drill 0.4) (layers F.Cu B.Cu) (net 27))
 (segment (start 152.282999 93.989999) (end 156.718 98.425) (width 0.25) (layer B.Cu) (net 27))
 (segment (start 156.718 99.440002) (end 165.608 108.330002) (width 0.25) (layer F.Cu) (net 27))
 (segment (start 156.718 98.425) (end 156.718 99.440002) (width 0.25) (layer F.Cu) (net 27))
 (segment (start 173.853001 121.929999) (end 171.958 123.825) (width 0.25) (layer F.Cu) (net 27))
 (segment (start 173.853001 108.284999) (end 173.853001 121.929999) (width 0.25) (layer F.Cu) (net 27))
 (segment (start 173.528001 107.959999) (end 173.853001 108.284999) (width 0.25) (layer F.Cu) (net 27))
 (segment (start 165.978003 107.959999) (end 173.528001 107.959999) (width 0.25) (layer F.Cu) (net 27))
 (segment (start 165.608 108.330002) (end 165.978003 107.959999) (width 0.25) (layer F.Cu) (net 27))
 (via (at 157.988 106.045) (size 0.6) (drill 0.4) (layers F.Cu B.Cu) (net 28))
 (segment (start 174.498 122.555) (end 157.988 106.045) (width 0.25) (layer B.Cu) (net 28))
 (segment (start 174.498 123.825) (end 174.498 122.555) (width 0.25) (layer B.Cu) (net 28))
 (segment (start 131.13501 74.22399) (end 129.794 75.565) (width 0.25) (layer F.Cu) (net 28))
 (segment (start 132.826338 74.22399) (end 131.13501 74.22399) (width 0.25) (layer F.Cu) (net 28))
 (segment (start 132.897348 74.295) (end 132.826338 74.22399) (width 0.25) (layer F.Cu) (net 28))
 (segment (start 133.858 74.295) (end 132.897348 74.295) (width 0.25) (layer F.Cu) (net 28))
 (segment (start 133.92901 74.22399) (end 133.858 74.295) (width 0.25) (layer F.Cu) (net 28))
 (segment (start 141.14261 74.920262) (end 140.446338 74.22399) (width 0.25) (layer F.Cu) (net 28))
 (segment (start 141.14261 76.046958) (end 141.14261 74.920262) (width 0.25) (layer F.Cu) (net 28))
 (segment (start 140.446338 74.22399) (end 133.92901 74.22399) (width 0.25) (layer F.Cu) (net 28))
 (segment (start 144.484012 76.90601) (end 142.001662 76.90601) (width 0.25) (layer F.Cu) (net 28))
 (segment (start 152.763001 85.184999) (end 144.484012 76.90601) (width 0.25) (layer F.Cu) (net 28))
 (segment (start 152.763001 86.265001) (end 152.763001 85.184999) (width 0.25) (layer F.Cu) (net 28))
 (segment (start 142.001662 76.90601) (end 141.14261 76.046958) (width 0.25) (layer F.Cu) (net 28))
 (segment (start 152.282999 86.745003) (end 152.763001 86.265001) (width 0.25) (layer F.Cu) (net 28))
 (segment (start 152.282999 100.339999) (end 152.282999 86.745003) (width 0.25) (layer F.Cu) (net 28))
 (segment (start 157.988 106.045) (end 152.282999 100.339999) (width 0.25) (layer F.Cu) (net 28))
 (via (at 173.228 108.585) (size 0.6) (drill 0.4) (layers F.Cu B.Cu) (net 14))
 (segment (start 177.038 108.585) (end 173.228 108.585) (width 0.25) (layer B.Cu) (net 14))
 (via (at 161.798 114.935) (size 0.6) (drill 0.4) (layers F.Cu B.Cu) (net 14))
 (segment (start 168.148 108.585) (end 161.798 114.935) (width 0.25) (layer F.Cu) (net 14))
 (segment (start 173.228 108.585) (end 168.148 108.585) (width 0.25) (layer F.Cu) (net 14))
 (segment (start 147.264652 123.825) (end 146.558 123.825) (width 0.25) (layer B.Cu) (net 14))
 (segment (start 156.154652 114.935) (end 147.264652 123.825) (width 0.25) (layer B.Cu) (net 14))
 (segment (start 161.798 114.935) (end 156.154652 114.935) (width 0.25) (layer B.Cu) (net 14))
 (segment (start 134.088 98.425) (end 133.858 98.655) (width 0.25) (layer F.Cu) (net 2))
 (segment (start 135.758 100.555) (end 138.163 100.555) (width 0.25) (layer F.Cu) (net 2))
 (segment (start 133.858 98.655) (end 135.758 100.555) (width 0.25) (layer F.Cu) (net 2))
 (via (at 127.508 98.425) (size 0.6) (drill 0.4) (layers F.Cu B.Cu) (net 2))
 (segment (start 127.738 98.655) (end 127.508 98.425) (width 0.25) (layer F.Cu) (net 2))
 (segment (start 133.858 98.655) (end 127.738 98.655) (width 0.25) (layer F.Cu) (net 2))
 (segment (start 127.508 98.425) (end 121.158 98.425) (width 0.25) (layer B.Cu) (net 2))
 (segment (start 123.698 95.885) (end 121.158 98.425) (width 0.25) (layer B.Cu) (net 2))
 (segment (start 123.698 92.075) (end 123.698 95.885) (width 0.25) (layer B.Cu) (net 2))
 (segment (start 140.028 90.985) (end 140.208 90.805) (width 0.25) (layer F.Cu) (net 4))
 (via (at 140.208 94.615) (size 0.6) (drill 0.4) (layers F.Cu B.Cu) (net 4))
 (segment (start 138.163 96.66) (end 140.208 94.615) (width 0.25) (layer F.Cu) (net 4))
 (segment (start 138.163 99.555) (end 138.163 96.66) (width 0.25) (layer F.Cu) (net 4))
 (via (at 142.748 92.075) (size 0.6) (drill 0.4) (layers F.Cu B.Cu) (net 4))
 (segment (start 140.208 94.615) (end 142.748 92.075) (width 0.25) (layer B.Cu) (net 4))
 (segment (start 141.478 90.805) (end 140.208 90.805) (width 0.25) (layer F.Cu) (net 4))
 (segment (start 142.748 92.075) (end 141.478 90.805) (width 0.25) (layer F.Cu) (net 4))
 (segment (start 136.398 86.995) (end 140.208 90.805) (width 0.25) (layer F.Cu) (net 4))
 (segment (start 144.018 86.995) (end 140.208 90.805) (width 0.25) (layer F.Cu) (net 4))
 (segment (start 144.018 85.725) (end 144.018 86.995) (width 0.25) (layer F.Cu) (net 4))
 (segment (start 132.588 90.958022) (end 132.588 90.805) (width 0.25) (layer F.Cu) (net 3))
 (segment (start 132.588 96.870002) (end 132.588 90.805) (width 0.25) (layer F.Cu) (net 3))
 (segment (start 132.797999 97.080001) (end 132.588 96.870002) (width 0.25) (layer F.Cu) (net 3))
 (segment (start 134.714979 97.080001) (end 132.797999 97.080001) (width 0.25) (layer F.Cu) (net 3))
 (segment (start 137.689978 100.055) (end 134.714979 97.080001) (width 0.25) (layer F.Cu) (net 3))
 (segment (start 138.163 100.055) (end 137.689978 100.055) (width 0.25) (layer F.Cu) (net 3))
 (segment (start 133.398 89.995) (end 132.588 90.805) (width 0.25) (layer F.Cu) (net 3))
 (segment (start 133.398 86.995) (end 133.398 89.995) (width 0.25) (layer F.Cu) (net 3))
 (segment (start 132.588 96.870002) (end 127.792998 96.870002) (width 0.25) (layer F.Cu) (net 3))
 (segment (start 121.158 103.505) (end 113.538 103.505) (width 0.25) (layer F.Cu) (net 3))
 (segment (start 127.792998 96.870002) (end 121.158 103.505) (width 0.25) (layer F.Cu) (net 3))
 (segment (start 151.638 96.115) (end 151.638 85.725) (width 0.25) (layer F.Cu) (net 5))
 (segment (start 146.558 101.195) (end 151.638 96.115) (width 0.25) (layer F.Cu) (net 5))
 (segment (start 161.798 116.435) (end 161.798 123.825) (width 0.25) (layer F.Cu) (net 5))
 (segment (start 146.558 101.195) (end 161.798 116.435) (width 0.25) (layer F.Cu) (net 5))
 (segment (start 147.590915 115.172085) (end 147.828 114.935) (width 0.25) (layer B.Cu) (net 11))
 (segment (start 132.60033 115.172085) (end 147.590915 115.172085) (width 0.25) (layer B.Cu) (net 11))
 (segment (start 131.720671 108.692914) (end 130.79567 109.617915) (width 0.25) (layer B.Cu) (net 12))
 (segment (start 133.443579 108.692914) (end 131.720671 108.692914) (width 0.25) (layer B.Cu) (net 12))
 (segment (start 134.605665 109.855) (end 133.443579 108.692914) (width 0.25) (layer B.Cu) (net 12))
 (segment (start 147.828 109.855) (end 134.605665 109.855) (width 0.25) (layer B.Cu) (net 12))
 (via (at 124.968 112.395) (size 0.6) (drill 0.4) (layers F.Cu B.Cu) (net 9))
 (segment (start 126.684333 114.111333) (end 124.968 112.395) (width 0.25) (layer B.Cu) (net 9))
 (segment (start 129.33567 114.111333) (end 126.684333 114.111333) (width 0.25) (layer B.Cu) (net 9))
 (via (at 128.778 99.695) (size 0.6) (drill 0.4) (layers F.Cu B.Cu) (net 9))
 (segment (start 128.778 108.585) (end 128.778 99.695) (width 0.25) (layer F.Cu) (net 9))
 (segment (start 124.968 112.395) (end 128.778 108.585) (width 0.25) (layer F.Cu) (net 9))
 (segment (start 128.778 99.695) (end 128.778 88.265) (width 0.25) (layer B.Cu) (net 9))
 (segment (start 124.968 85.725) (end 123.698 84.455) (width 0.25) (layer B.Cu) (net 7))
 (segment (start 128.778 85.725) (end 124.968 85.725) (width 0.25) (layer B.Cu) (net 7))
 (segment (start 137.538 91.945) (end 137.538 106.045) (width 0.25) (layer B.Cu) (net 10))
 (via (at 137.538 106.045) (size 0.6) (drill 0.4) (layers F.Cu B.Cu) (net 10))
 (segment (start 128.778 83.185) (end 137.538 91.945) (width 0.25) (layer B.Cu) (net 10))
 (segment (start 135.229335 110.678667) (end 134.06033 110.678667) (width 0.25) (layer F.Cu) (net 10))
 (segment (start 137.538 108.370002) (end 135.229335 110.678667) (width 0.25) (layer F.Cu) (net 10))
 (segment (start 137.538 106.045) (end 137.538 108.370002) (width 0.25) (layer F.Cu) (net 10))
 (via (at 136.398 108.585) (size 0.6) (drill 0.4) (layers F.Cu B.Cu) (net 8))
 (segment (start 135.365085 109.617915) (end 136.398 108.585) (width 0.25) (layer F.Cu) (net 8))
 (segment (start 132.60033 109.617915) (end 135.365085 109.617915) (width 0.25) (layer F.Cu) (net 8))
 (segment (start 145.288 99.695) (end 161.798 99.695) (width 0.25) (layer B.Cu) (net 8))
 (segment (start 136.398 108.585) (end 145.288 99.695) (width 0.25) (layer B.Cu) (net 8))
 (segment (start 151.528999 84.599999) (end 154.322999 84.599999) (width 0.25) (layer B.Cu) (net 15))
 (segment (start 142.494 75.565) (end 151.528999 84.599999) (width 0.25) (layer B.Cu) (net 15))
 (segment (start 175.768 106.045) (end 177.038 106.045) (width 0.25) (layer B.Cu) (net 15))
 (segment (start 154.322999 84.599999) (end 175.768 106.045) (width 0.25) (layer B.Cu) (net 15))
 (segment (start 152.352989 84.149989) (end 156.412989 84.149989) (width 0.25) (layer B.Cu) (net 18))
 (segment (start 145.034 76.831) (end 152.352989 84.149989) (width 0.25) (layer B.Cu) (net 18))
 (segment (start 145.034 75.565) (end 145.034 76.831) (width 0.25) (layer B.Cu) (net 18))
 (segment (start 170.688 98.425) (end 177.038 98.425) (width 0.25) (layer B.Cu) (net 18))
 (segment (start 156.412989 84.149989) (end 170.688 98.425) (width 0.25) (layer B.Cu) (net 18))
 (segment (start 158.05901 76.90601) (end 177.038 95.885) (width 0.25) (layer B.Cu) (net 19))
 (segment (start 148.91501 76.90601) (end 158.05901 76.90601) (width 0.25) (layer B.Cu) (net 19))
 (segment (start 147.574 75.565) (end 148.91501 76.90601) (width 0.25) (layer B.Cu) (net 19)))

